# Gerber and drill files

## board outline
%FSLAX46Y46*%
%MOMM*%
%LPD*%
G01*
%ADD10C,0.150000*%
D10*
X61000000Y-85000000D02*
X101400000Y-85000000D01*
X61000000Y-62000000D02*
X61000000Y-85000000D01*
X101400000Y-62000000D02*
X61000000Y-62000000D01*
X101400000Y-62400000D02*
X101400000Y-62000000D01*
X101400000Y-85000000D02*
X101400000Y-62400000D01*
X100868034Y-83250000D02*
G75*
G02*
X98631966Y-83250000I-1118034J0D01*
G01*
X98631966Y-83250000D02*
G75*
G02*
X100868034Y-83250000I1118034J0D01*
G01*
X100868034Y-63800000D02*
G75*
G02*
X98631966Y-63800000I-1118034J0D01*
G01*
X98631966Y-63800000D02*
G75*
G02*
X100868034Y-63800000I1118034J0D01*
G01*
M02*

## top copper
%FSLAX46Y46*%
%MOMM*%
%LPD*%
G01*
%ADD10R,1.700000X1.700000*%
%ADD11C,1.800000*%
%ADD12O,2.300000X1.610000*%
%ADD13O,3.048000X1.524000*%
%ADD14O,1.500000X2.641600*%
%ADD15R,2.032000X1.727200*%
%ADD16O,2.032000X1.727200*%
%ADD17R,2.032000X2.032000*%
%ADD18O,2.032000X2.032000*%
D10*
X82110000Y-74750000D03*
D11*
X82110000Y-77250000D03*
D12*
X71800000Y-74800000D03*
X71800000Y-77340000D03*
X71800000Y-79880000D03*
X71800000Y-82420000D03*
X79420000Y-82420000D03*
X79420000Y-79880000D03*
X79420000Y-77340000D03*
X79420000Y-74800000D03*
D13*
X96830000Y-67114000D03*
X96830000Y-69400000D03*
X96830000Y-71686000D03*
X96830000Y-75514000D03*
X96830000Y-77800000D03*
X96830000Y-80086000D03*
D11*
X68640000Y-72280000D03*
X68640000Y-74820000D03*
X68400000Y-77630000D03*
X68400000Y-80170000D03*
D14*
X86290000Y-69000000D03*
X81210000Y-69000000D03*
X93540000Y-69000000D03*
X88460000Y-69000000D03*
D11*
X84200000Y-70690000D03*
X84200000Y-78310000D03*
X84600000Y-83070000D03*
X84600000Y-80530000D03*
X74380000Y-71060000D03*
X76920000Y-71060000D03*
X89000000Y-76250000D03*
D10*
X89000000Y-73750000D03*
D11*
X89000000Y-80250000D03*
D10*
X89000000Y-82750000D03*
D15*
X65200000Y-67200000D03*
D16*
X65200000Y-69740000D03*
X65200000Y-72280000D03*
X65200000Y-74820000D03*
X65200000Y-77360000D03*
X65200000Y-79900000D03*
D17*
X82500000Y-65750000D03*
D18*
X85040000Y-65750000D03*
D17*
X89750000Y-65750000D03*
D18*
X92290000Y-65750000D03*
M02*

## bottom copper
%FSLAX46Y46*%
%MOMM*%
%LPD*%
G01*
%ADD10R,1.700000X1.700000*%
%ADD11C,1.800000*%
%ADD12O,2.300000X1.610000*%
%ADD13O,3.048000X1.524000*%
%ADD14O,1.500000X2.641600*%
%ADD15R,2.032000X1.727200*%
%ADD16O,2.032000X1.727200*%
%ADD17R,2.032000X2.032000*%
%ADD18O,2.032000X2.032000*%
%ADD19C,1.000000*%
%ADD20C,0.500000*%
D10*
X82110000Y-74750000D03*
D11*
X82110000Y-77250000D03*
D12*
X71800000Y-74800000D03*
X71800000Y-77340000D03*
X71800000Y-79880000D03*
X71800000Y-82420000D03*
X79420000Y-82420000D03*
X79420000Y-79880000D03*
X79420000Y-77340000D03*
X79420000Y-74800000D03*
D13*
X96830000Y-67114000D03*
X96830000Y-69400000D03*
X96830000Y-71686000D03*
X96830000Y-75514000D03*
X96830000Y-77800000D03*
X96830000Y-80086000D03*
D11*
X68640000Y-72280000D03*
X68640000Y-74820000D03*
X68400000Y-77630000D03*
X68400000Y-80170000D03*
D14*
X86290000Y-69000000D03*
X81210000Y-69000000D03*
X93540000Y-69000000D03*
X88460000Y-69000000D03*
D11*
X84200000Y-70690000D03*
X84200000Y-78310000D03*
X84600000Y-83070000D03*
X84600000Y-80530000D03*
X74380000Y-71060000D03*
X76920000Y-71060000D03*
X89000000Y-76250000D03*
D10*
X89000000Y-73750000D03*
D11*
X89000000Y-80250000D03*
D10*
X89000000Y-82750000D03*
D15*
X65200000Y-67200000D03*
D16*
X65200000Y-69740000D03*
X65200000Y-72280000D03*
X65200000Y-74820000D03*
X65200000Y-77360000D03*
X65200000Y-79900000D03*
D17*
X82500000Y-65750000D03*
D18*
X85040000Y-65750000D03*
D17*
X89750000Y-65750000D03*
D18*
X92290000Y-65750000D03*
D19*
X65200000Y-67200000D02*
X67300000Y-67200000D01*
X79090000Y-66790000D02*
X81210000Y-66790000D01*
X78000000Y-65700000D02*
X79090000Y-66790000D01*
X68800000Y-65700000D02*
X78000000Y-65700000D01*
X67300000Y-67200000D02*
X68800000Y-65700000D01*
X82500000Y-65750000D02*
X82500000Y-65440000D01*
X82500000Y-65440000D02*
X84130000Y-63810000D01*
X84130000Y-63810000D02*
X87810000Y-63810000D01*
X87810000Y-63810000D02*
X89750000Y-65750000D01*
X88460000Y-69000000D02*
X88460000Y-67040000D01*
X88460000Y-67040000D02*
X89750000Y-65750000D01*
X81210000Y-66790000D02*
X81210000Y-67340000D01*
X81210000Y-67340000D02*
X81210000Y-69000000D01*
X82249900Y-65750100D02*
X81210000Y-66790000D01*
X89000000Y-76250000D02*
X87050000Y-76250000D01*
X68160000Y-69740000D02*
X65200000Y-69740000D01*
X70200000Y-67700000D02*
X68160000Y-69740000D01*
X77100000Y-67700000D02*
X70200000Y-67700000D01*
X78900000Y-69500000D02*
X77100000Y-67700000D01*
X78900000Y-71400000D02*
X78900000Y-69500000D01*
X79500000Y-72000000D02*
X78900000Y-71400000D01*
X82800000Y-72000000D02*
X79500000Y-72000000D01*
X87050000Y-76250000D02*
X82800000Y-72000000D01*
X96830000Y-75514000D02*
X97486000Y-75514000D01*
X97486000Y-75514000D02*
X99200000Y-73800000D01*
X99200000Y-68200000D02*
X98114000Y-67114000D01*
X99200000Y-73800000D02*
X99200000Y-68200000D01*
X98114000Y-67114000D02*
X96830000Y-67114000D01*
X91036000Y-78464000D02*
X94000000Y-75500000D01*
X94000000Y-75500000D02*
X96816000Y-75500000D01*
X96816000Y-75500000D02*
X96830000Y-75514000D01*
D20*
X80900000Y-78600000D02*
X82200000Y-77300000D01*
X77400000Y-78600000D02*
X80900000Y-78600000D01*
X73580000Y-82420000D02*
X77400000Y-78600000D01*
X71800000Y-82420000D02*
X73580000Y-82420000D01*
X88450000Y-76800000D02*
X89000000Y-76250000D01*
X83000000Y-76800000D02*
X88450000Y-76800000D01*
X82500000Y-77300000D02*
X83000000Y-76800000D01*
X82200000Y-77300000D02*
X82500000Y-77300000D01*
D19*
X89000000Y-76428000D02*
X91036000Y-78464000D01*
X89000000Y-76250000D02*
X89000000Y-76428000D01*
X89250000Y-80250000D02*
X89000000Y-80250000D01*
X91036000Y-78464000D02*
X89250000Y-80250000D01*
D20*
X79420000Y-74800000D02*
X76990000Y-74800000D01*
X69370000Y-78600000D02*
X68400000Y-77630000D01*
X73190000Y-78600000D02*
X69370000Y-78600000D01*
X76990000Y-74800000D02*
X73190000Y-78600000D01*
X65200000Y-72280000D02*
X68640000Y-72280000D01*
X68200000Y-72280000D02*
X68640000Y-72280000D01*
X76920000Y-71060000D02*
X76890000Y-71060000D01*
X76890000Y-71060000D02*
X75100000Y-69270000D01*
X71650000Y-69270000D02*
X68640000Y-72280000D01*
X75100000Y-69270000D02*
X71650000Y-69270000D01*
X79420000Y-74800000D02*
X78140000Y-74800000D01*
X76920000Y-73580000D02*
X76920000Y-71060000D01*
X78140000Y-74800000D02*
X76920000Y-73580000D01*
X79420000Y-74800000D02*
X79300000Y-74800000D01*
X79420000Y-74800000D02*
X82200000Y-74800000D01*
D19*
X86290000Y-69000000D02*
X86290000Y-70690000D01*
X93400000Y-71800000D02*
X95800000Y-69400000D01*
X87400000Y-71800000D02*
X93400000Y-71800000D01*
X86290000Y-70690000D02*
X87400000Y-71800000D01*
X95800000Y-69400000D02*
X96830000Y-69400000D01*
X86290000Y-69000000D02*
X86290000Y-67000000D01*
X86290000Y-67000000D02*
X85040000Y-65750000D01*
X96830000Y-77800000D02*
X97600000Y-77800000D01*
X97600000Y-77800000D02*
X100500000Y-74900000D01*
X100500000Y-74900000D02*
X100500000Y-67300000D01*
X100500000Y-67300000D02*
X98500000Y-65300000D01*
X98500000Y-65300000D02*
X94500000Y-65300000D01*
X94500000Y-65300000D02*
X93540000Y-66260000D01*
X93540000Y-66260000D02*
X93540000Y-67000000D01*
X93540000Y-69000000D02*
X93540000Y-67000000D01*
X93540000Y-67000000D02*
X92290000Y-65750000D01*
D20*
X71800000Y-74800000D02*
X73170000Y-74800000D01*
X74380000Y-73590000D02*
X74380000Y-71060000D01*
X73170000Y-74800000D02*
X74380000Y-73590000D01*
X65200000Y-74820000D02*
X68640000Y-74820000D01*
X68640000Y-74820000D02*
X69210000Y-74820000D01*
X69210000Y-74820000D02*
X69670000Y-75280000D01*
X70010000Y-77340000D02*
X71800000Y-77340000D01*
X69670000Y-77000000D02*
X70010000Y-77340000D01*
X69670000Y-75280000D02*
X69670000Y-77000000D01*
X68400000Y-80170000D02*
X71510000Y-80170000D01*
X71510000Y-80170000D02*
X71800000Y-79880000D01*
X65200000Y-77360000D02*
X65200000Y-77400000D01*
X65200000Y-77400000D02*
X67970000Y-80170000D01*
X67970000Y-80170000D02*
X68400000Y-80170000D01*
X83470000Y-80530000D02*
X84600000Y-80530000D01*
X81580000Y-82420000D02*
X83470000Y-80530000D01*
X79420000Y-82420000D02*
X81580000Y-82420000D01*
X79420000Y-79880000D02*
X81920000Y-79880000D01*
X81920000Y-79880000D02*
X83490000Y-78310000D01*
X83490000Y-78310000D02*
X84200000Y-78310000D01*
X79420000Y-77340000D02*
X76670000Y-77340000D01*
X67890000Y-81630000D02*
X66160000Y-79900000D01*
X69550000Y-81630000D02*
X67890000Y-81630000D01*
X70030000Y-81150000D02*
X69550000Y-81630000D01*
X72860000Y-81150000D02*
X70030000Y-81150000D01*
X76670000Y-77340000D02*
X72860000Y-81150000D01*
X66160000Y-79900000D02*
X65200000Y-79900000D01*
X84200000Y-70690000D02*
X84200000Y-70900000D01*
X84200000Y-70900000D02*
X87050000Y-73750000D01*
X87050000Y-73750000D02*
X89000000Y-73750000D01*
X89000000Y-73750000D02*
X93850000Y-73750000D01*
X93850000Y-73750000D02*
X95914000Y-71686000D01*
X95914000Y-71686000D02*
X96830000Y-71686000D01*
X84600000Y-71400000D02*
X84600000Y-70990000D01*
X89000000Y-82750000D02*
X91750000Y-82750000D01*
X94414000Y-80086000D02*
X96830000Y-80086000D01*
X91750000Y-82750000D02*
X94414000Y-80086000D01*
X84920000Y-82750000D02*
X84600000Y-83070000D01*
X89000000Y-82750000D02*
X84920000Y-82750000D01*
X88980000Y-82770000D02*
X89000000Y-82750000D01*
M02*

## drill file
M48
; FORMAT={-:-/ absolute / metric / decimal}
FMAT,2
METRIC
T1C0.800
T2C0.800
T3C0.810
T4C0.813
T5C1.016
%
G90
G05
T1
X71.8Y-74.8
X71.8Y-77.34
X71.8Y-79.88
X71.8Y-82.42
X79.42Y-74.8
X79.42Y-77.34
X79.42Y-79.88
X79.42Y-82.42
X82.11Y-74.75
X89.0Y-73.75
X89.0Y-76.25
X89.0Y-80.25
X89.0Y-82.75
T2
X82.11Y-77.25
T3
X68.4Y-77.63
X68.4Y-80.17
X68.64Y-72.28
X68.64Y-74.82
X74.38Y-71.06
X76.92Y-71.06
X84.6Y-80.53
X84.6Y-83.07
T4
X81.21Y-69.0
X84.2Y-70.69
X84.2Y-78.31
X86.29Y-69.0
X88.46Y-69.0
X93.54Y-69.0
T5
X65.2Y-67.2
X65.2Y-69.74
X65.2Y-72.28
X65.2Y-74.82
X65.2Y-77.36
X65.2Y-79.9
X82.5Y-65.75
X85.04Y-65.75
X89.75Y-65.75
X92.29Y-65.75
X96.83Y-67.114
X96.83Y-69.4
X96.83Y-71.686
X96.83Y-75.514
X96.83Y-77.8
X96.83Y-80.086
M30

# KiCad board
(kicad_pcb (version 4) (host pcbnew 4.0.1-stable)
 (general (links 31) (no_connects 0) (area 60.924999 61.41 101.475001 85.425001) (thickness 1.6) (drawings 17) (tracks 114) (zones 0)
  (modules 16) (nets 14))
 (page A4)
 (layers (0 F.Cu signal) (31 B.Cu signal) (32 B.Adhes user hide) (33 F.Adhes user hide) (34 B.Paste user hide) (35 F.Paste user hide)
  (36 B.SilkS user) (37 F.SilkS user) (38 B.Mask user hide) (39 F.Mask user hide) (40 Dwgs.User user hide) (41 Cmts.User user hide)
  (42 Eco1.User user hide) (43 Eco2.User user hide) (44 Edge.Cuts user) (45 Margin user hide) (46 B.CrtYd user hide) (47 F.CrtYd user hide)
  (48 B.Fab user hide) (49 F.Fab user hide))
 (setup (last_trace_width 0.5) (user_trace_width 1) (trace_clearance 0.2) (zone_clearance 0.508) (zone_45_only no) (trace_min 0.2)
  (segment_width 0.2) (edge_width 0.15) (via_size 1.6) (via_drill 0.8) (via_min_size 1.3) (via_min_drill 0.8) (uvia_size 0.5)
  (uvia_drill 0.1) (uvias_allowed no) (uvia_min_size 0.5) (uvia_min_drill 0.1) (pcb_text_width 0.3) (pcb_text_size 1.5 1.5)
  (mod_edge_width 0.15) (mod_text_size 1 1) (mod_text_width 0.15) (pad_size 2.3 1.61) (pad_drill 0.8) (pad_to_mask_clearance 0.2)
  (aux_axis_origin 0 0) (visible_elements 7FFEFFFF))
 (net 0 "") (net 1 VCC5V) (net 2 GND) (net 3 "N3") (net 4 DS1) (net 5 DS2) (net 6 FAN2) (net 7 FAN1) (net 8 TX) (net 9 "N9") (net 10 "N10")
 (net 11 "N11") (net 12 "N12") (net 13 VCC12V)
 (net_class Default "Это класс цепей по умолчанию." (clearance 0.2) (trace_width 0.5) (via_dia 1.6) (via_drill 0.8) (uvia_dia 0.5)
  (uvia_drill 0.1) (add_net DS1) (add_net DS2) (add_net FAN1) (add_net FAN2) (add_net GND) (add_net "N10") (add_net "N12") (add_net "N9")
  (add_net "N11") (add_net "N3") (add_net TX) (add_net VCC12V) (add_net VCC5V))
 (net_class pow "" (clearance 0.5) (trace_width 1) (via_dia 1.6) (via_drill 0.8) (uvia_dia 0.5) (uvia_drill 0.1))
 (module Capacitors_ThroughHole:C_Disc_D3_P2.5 (layer F.Cu) (at 82.11 74.75 270)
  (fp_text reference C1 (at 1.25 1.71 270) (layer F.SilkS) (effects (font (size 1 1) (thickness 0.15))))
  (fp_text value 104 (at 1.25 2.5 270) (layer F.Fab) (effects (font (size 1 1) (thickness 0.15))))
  (pad 1 thru_hole rect (at 0 0 270) (size 1.7 1.7) (drill 0.8) (layers *.Cu *.Mask F.SilkS) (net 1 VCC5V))
  (pad 2 thru_hole circle (at 2.5 0 270) (size 1.8 1.8) (drill 0.8001) (layers *.Cu *.Mask F.SilkS) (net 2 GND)))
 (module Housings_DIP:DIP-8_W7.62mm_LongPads (layer F.Cu) (at 71.8 74.8)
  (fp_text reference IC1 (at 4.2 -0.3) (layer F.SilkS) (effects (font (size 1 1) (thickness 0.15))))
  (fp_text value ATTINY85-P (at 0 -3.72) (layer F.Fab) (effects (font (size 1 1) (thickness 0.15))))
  (pad 1 thru_hole oval (at 0 0) (size 2.3 1.61) (drill 0.8) (layers *.Cu *.Mask F.SilkS) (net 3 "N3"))
  (pad 2 thru_hole oval (at 0 2.54) (size 2.3 1.61) (drill 0.8) (layers *.Cu *.Mask F.SilkS) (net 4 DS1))
  (pad 3 thru_hole oval (at 0 5.08) (size 2.3 1.61) (drill 0.8) (layers *.Cu *.Mask F.SilkS) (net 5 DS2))
  (pad 4 thru_hole oval (at 0 7.62) (size 2.3 1.61) (drill 0.8) (layers *.Cu *.Mask F.SilkS) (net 2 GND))
  (pad 5 thru_hole oval (at 7.62 7.62) (size 2.3 1.61) (drill 0.8) (layers *.Cu *.Mask F.SilkS) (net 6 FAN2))
  (pad 6 thru_hole oval (at 7.62 5.08) (size 2.3 1.61) (drill 0.8) (layers *.Cu *.Mask F.SilkS) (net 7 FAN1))
  (pad 7 thru_hole oval (at 7.62 2.54) (size 2.3 1.61) (drill 0.8) (layers *.Cu *.Mask F.SilkS) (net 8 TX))
  (pad 8 thru_hole oval (at 7.62 0) (size 2.3 1.61) (drill 0.8) (layers *.Cu *.Mask F.SilkS) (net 1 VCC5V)))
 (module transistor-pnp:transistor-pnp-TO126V (layer F.Cu) (at 98.1 69.4 270)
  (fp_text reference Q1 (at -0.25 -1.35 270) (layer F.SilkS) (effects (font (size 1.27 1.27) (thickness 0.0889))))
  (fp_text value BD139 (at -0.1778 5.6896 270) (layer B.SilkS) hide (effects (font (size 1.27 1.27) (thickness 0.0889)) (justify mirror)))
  (pad 1 thru_hole oval (at -2.286 1.27 270) (size 1.524 3.048) (drill 1.016) (layers *.Cu F.Paste F.SilkS F.Mask) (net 2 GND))
  (pad 2 thru_hole oval (at 0 1.27 270) (size 1.524 3.048) (drill 1.016) (layers *.Cu F.Paste F.SilkS F.Mask) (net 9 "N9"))
  (pad 3 thru_hole oval (at 2.286 1.27 270) (size 1.524 3.048) (drill 1.016) (layers *.Cu F.Paste F.SilkS F.Mask) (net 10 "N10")))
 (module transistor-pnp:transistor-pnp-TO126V (layer F.Cu) (at 98.1 77.8 270)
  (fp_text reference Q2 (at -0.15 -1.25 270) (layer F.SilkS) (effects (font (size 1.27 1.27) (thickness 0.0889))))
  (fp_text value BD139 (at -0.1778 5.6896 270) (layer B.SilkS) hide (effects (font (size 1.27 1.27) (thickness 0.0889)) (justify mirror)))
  (pad 1 thru_hole oval (at -2.286 1.27 270) (size 1.524 3.048) (drill 1.016) (layers *.Cu F.Paste F.SilkS F.Mask) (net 2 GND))
  (pad 2 thru_hole oval (at 0 1.27 270) (size 1.524 3.048) (drill 1.016) (layers *.Cu F.Paste F.SilkS F.Mask) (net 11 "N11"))
  (pad 3 thru_hole oval (at 2.286 1.27 270) (size 1.524 3.048) (drill 1.016) (layers *.Cu F.Paste F.SilkS F.Mask) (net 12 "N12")))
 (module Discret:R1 (layer F.Cu) (at 68.64 73.55 270)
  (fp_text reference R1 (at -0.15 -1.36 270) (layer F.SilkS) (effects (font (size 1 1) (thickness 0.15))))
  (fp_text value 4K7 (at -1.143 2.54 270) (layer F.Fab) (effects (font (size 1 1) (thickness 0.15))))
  (pad 1 thru_hole circle (at -1.27 0 270) (size 1.8 1.8) (drill 0.81) (layers *.Cu *.Mask F.SilkS) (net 1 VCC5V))
  (pad 2 thru_hole circle (at 1.27 0 270) (size 1.8 1.8) (drill 0.81) (layers *.Cu *.Mask F.SilkS) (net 4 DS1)))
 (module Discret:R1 (layer F.Cu) (at 68.4 78.9 270)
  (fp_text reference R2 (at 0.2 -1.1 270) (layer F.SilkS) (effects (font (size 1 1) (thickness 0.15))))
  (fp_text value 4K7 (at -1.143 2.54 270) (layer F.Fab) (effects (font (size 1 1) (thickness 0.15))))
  (pad 1 thru_hole circle (at -1.27 0 270) (size 1.8 1.8) (drill 0.81) (layers *.Cu *.Mask F.SilkS) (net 1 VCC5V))
  (pad 2 thru_hole circle (at 1.27 0 270) (size 1.8 1.8) (drill 0.81) (layers *.Cu *.Mask F.SilkS) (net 5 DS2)))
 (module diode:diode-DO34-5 (layer F.Cu) (at 83.75 69)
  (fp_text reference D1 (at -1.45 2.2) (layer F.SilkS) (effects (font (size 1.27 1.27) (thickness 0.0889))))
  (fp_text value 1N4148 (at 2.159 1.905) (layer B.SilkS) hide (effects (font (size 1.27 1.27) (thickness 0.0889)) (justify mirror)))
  (pad 2 thru_hole oval (at 2.54 0) (size 1.5 2.6416) (drill 0.8128) (layers *.Cu F.Paste F.SilkS F.Mask) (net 9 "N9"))
  (pad 1 thru_hole oval (at -2.54 0) (size 1.5 2.6416) (drill 0.8128) (layers *.Cu F.Paste F.SilkS F.Mask) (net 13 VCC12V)))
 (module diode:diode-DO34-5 (layer F.Cu) (at 91 69)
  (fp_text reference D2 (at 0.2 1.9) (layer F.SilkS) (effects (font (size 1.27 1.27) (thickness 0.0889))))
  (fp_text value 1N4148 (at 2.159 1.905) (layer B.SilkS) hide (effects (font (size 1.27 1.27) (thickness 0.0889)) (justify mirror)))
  (pad 2 thru_hole oval (at 2.54 0) (size 1.5 2.6416) (drill 0.8128) (layers *.Cu F.Paste F.SilkS F.Mask) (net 11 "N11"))
  (pad 1 thru_hole oval (at -2.54 0) (size 1.5 2.6416) (drill 0.8128) (layers *.Cu F.Paste F.SilkS F.Mask) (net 13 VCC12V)))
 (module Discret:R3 (layer F.Cu) (at 84.2 74.5 270)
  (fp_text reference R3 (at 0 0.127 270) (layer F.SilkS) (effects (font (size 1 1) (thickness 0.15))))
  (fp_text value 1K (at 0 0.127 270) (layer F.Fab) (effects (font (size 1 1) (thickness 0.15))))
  (pad 1 thru_hole circle (at -3.81 0 270) (size 1.8 1.8) (drill 0.8128) (layers *.Cu *.Mask F.SilkS) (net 10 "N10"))
  (pad 2 thru_hole circle (at 3.81 0 270) (size 1.8 1.8) (drill 0.8128) (layers *.Cu *.Mask F.SilkS) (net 7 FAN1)))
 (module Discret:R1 (layer F.Cu) (at 84.6 81.8 90)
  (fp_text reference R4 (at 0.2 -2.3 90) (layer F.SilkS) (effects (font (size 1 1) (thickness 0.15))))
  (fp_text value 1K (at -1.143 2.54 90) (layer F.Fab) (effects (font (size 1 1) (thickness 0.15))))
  (pad 1 thru_hole circle (at -1.27 0 90) (size 1.8 1.8) (drill 0.81) (layers *.Cu *.Mask F.SilkS) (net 12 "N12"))
  (pad 2 thru_hole circle (at 1.27 0 90) (size 1.8 1.8) (drill 0.81) (layers *.Cu *.Mask F.SilkS) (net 6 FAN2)))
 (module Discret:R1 (layer F.Cu) (at 75.65 71.06)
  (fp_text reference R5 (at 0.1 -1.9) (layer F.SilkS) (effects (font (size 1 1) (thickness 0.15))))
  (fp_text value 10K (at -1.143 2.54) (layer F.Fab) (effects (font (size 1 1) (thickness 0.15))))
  (pad 1 thru_hole circle (at -1.27 0) (size 1.8 1.8) (drill 0.81) (layers *.Cu *.Mask F.SilkS) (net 3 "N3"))
  (pad 2 thru_hole circle (at 1.27 0) (size 1.8 1.8) (drill 0.81) (layers *.Cu *.Mask F.SilkS) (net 1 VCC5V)))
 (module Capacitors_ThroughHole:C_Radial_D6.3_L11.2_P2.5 (layer F.Cu) (at 89 73.75 270)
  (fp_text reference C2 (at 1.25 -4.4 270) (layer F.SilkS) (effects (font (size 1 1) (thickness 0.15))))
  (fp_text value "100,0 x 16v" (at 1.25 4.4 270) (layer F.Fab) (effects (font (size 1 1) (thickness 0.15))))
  (pad 2 thru_hole circle (at 2.5 0 270) (size 1.8 1.8) (drill 0.8) (layers *.Cu *.Mask F.SilkS) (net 2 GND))
  (pad 1 thru_hole rect (at 0 0 270) (size 1.7 1.7) (drill 0.8) (layers *.Cu *.Mask F.SilkS) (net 10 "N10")))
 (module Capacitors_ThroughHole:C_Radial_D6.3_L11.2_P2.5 (layer F.Cu) (at 89 82.75 90)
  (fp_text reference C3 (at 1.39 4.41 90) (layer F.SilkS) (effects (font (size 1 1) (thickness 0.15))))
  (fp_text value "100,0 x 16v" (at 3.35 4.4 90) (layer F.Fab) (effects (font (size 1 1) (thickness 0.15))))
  (pad 2 thru_hole circle (at 2.5 0 90) (size 1.8 1.8) (drill 0.8) (layers *.Cu *.Mask F.SilkS) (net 2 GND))
  (pad 1 thru_hole rect (at 0 0 90) (size 1.7 1.7) (drill 0.8) (layers *.Cu *.Mask F.SilkS) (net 12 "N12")))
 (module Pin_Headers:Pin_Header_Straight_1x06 (layer F.Cu) (at 65.2 67.2)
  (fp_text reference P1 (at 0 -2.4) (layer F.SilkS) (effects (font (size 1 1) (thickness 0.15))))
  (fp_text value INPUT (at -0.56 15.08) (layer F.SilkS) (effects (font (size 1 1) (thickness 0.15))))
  (pad 1 thru_hole rect (at 0 0) (size 2.032 1.7272) (drill 1.016) (layers *.Cu *.Mask F.SilkS) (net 13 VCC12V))
  (pad 2 thru_hole oval (at 0 2.54) (size 2.032 1.7272) (drill 1.016) (layers *.Cu *.Mask F.SilkS) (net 2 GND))
  (pad 3 thru_hole oval (at 0 5.08) (size 2.032 1.7272) (drill 1.016) (layers *.Cu *.Mask F.SilkS) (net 1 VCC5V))
  (pad 4 thru_hole oval (at 0 7.62) (size 2.032 1.7272) (drill 1.016) (layers *.Cu *.Mask F.SilkS) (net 4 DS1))
  (pad 5 thru_hole oval (at 0 10.16) (size 2.032 1.7272) (drill 1.016) (layers *.Cu *.Mask F.SilkS) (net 5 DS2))
  (pad 6 thru_hole oval (at 0 12.7) (size 2.032 1.7272) (drill 1.016) (layers *.Cu *.Mask F.SilkS) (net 8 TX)))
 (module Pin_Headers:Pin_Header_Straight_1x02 (layer F.Cu) (at 82.5 65.75 90)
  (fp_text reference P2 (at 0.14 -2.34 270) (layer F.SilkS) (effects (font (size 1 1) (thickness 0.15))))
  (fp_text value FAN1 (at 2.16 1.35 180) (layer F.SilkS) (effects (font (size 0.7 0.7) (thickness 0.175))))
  (pad 1 thru_hole rect (at 0 0 90) (size 2.032 2.032) (drill 1.016) (layers *.Cu *.Mask F.SilkS) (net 13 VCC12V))
  (pad 2 thru_hole oval (at 0 2.54 90) (size 2.032 2.032) (drill 1.016) (layers *.Cu *.Mask F.SilkS) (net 9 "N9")))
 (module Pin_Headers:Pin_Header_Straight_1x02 (layer F.Cu) (at 89.75 65.75 90)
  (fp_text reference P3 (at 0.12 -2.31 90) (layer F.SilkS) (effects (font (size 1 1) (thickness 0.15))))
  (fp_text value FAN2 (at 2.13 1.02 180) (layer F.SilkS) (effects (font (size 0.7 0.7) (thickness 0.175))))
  (pad 1 thru_hole rect (at 0 0 90) (size 2.032 2.032) (drill 1.016) (layers *.Cu *.Mask F.SilkS) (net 13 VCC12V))
  (pad 2 thru_hole oval (at 0 2.54 90) (size 2.032 2.032) (drill 1.016) (layers *.Cu *.Mask F.SilkS) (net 11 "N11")))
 (gr_line (start 61 85) (end 101.4 85) (angle 90) (layer Edge.Cuts) (width 0.15))
 (gr_line (start 61 62) (end 61 85) (angle 90) (layer Edge.Cuts) (width 0.15))
 (gr_line (start 101.4 62) (end 61 62) (angle 90) (layer Edge.Cuts) (width 0.15))
 (gr_line (start 101.4 62.4) (end 101.4 62) (angle 90) (layer Edge.Cuts) (width 0.15))
 (gr_line (start 101.4 85) (end 101.4 62.4) (angle 90) (layer Edge.Cuts) (width 0.15))
 (gr_circle (center 99.75 83.25) (end 100.75 82.75) (layer Edge.Cuts) (width 0.15))
 (gr_circle (center 99.75 63.8) (end 100.75 63.3) (layer Edge.Cuts) (width 0.15))
 (segment (start 65.2 67.2) (end 67.3 67.2) (width 1) (layer B.Cu) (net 13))
 (segment (start 79.09 66.79) (end 81.21 66.79) (width 1) (layer B.Cu) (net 13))
 (segment (start 78 65.7) (end 79.09 66.79) (width 1) (layer B.Cu) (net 13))
 (segment (start 68.8 65.7) (end 78 65.7) (width 1) (layer B.Cu) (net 13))
 (segment (start 67.3 67.2) (end 68.8 65.7) (width 1) (layer B.Cu) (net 13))
 (segment (start 82.5 65.75) (end 82.5 65.44) (width 1) (layer B.Cu) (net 13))
 (segment (start 82.5 65.44) (end 84.13 63.81) (width 1) (layer B.Cu) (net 13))
 (segment (start 84.13 63.81) (end 87.81 63.81) (width 1) (layer B.Cu) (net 13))
 (segment (start 87.81 63.81) (end 89.75 65.75) (width 1) (layer B.Cu) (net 13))
 (segment (start 88.46 69) (end 88.46 67.04) (width 1) (layer B.Cu) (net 13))
 (segment (start 88.46 67.04) (end 89.75 65.75) (width 1) (layer B.Cu) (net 13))
 (segment (start 81.21 66.79) (end 81.21 67.34) (width 1) (layer B.Cu) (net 13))
 (segment (start 81.21 67.34) (end 81.21 69) (width 1) (layer B.Cu) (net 13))
 (segment (start 82.2499 65.7501) (end 81.21 66.79) (width 1) (layer B.Cu) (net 13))
 (segment (start 89 76.25) (end 87.05 76.25) (width 1) (layer B.Cu) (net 2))
 (segment (start 68.16 69.74) (end 65.2 69.74) (width 1) (layer B.Cu) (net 2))
 (segment (start 70.2 67.7) (end 68.16 69.74) (width 1) (layer B.Cu) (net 2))
 (segment (start 77.1 67.7) (end 70.2 67.7) (width 1) (layer B.Cu) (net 2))
 (segment (start 78.9 69.5) (end 77.1 67.7) (width 1) (layer B.Cu) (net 2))
 (segment (start 78.9 71.4) (end 78.9 69.5) (width 1) (layer B.Cu) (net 2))
 (segment (start 79.5 72) (end 78.9 71.4) (width 1) (layer B.Cu) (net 2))
 (segment (start 82.8 72) (end 79.5 72) (width 1) (layer B.Cu) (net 2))
 (segment (start 87.05 76.25) (end 82.8 72) (width 1) (layer B.Cu) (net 2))
 (segment (start 96.83 75.514) (end 97.486 75.514) (width 1) (layer B.Cu) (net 2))
 (segment (start 97.486 75.514) (end 99.2 73.8) (width 1) (layer B.Cu) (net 2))
 (segment (start 99.2 68.2) (end 98.114 67.114) (width 1) (layer B.Cu) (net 2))
 (segment (start 99.2 73.8) (end 99.2 68.2) (width 1) (layer B.Cu) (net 2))
 (segment (start 98.114 67.114) (end 96.83 67.114) (width 1) (layer B.Cu) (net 2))
 (segment (start 91.036 78.464) (end 94 75.5) (width 1) (layer B.Cu) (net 2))
 (segment (start 94 75.5) (end 96.816 75.5) (width 1) (layer B.Cu) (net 2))
 (segment (start 96.816 75.5) (end 96.83 75.514) (width 1) (layer B.Cu) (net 2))
 (segment (start 80.9 78.6) (end 82.2 77.3) (width 0.5) (layer B.Cu) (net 2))
 (segment (start 77.4 78.6) (end 80.9 78.6) (width 0.5) (layer B.Cu) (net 2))
 (segment (start 73.58 82.42) (end 77.4 78.6) (width 0.5) (layer B.Cu) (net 2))
 (segment (start 71.8 82.42) (end 73.58 82.42) (width 0.5) (layer B.Cu) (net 2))
 (segment (start 88.45 76.8) (end 89 76.25) (width 0.5) (layer B.Cu) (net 2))
 (segment (start 83 76.8) (end 88.45 76.8) (width 0.5) (layer B.Cu) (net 2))
 (segment (start 82.5 77.3) (end 83 76.8) (width 0.5) (layer B.Cu) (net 2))
 (segment (start 82.2 77.3) (end 82.5 77.3) (width 0.5) (layer B.Cu) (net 2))
 (segment (start 89 76.428) (end 91.036 78.464) (width 1) (layer B.Cu) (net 2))
 (segment (start 89 76.25) (end 89 76.428) (width 1) (layer B.Cu) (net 2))
 (segment (start 89.25 80.25) (end 89 80.25) (width 1) (layer B.Cu) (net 2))
 (segment (start 91.036 78.464) (end 89.25 80.25) (width 1) (layer B.Cu) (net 2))
 (segment (start 79.42 74.8) (end 76.99 74.8) (width 0.5) (layer B.Cu) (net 1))
 (segment (start 69.37 78.6) (end 68.4 77.63) (width 0.5) (layer B.Cu) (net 1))
 (segment (start 73.19 78.6) (end 69.37 78.6) (width 0.5) (layer B.Cu) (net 1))
 (segment (start 76.99 74.8) (end 73.19 78.6) (width 0.5) (layer B.Cu) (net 1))
 (segment (start 65.2 72.28) (end 68.64 72.28) (width 0.5) (layer B.Cu) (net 1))
 (segment (start 68.2 72.28) (end 68.64 72.28) (width 0.5) (layer B.Cu) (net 1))
 (segment (start 76.92 71.06) (end 76.89 71.06) (width 0.5) (layer B.Cu) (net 1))
 (segment (start 76.89 71.06) (end 75.1 69.27) (width 0.5) (layer B.Cu) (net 1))
 (segment (start 71.65 69.27) (end 68.64 72.28) (width 0.5) (layer B.Cu) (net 1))
 (segment (start 75.1 69.27) (end 71.65 69.27) (width 0.5) (layer B.Cu) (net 1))
 (segment (start 79.42 74.8) (end 78.14 74.8) (width 0.5) (layer B.Cu) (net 1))
 (segment (start 76.92 73.58) (end 76.92 71.06) (width 0.5) (layer B.Cu) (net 1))
 (segment (start 78.14 74.8) (end 76.92 73.58) (width 0.5) (layer B.Cu) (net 1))
 (segment (start 79.42 74.8) (end 79.3 74.8) (width 0.5) (layer B.Cu) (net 1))
 (segment (start 79.42 74.8) (end 82.2 74.8) (width 0.5) (layer B.Cu) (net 1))
 (segment (start 86.29 69) (end 86.29 70.69) (width 1) (layer B.Cu) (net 9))
 (segment (start 93.4 71.8) (end 95.8 69.4) (width 1) (layer B.Cu) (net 9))
 (segment (start 87.4 71.8) (end 93.4 71.8) (width 1) (layer B.Cu) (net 9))
 (segment (start 86.29 70.69) (end 87.4 71.8) (width 1) (layer B.Cu) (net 9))
 (segment (start 95.8 69.4) (end 96.83 69.4) (width 1) (layer B.Cu) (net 9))
 (segment (start 86.29 69) (end 86.29 67) (width 1) (layer B.Cu) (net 9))
 (segment (start 86.29 67) (end 85.04 65.75) (width 1) (layer B.Cu) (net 9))
 (segment (start 96.83 77.8) (end 97.6 77.8) (width 1) (layer B.Cu) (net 11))
 (segment (start 97.6 77.8) (end 100.5 74.9) (width 1) (layer B.Cu) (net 11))
 (segment (start 100.5 74.9) (end 100.5 67.3) (width 1) (layer B.Cu) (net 11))
 (segment (start 100.5 67.3) (end 98.5 65.3) (width 1) (layer B.Cu) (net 11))
 (segment (start 98.5 65.3) (end 94.5 65.3) (width 1) (layer B.Cu) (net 11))
 (segment (start 94.5 65.3) (end 93.54 66.26) (width 1) (layer B.Cu) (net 11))
 (segment (start 93.54 66.26) (end 93.54 67) (width 1) (layer B.Cu) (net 11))
 (segment (start 93.54 69) (end 93.54 67) (width 1) (layer B.Cu) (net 11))
 (segment (start 93.54 67) (end 92.29 65.75) (width 1) (layer B.Cu) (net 11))
 (segment (start 71.8 74.8) (end 73.17 74.8) (width 0.5) (layer B.Cu) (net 3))
 (segment (start 74.38 73.59) (end 74.38 71.06) (width 0.5) (layer B.Cu) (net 3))
 (segment (start 73.17 74.8) (end 74.38 73.59) (width 0.5) (layer B.Cu) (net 3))
 (segment (start 65.2 74.82) (end 68.64 74.82) (width 0.5) (layer B.Cu) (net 4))
 (segment (start 68.64 74.82) (end 69.21 74.82) (width 0.5) (layer B.Cu) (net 4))
 (segment (start 69.21 74.82) (end 69.67 75.28) (width 0.5) (layer B.Cu) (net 4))
 (segment (start 70.01 77.34) (end 71.8 77.34) (width 0.5) (layer B.Cu) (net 4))
 (segment (start 69.67 77) (end 70.01 77.34) (width 0.5) (layer B.Cu) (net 4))
 (segment (start 69.67 75.28) (end 69.67 77) (width 0.5) (layer B.Cu) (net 4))
 (segment (start 68.4 80.17) (end 71.51 80.17) (width 0.5) (layer B.Cu) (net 5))
 (segment (start 71.51 80.17) (end 71.8 79.88) (width 0.5) (layer B.Cu) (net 5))
 (segment (start 65.2 77.36) (end 65.2 77.4) (width 0.5) (layer B.Cu) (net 5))
 (segment (start 65.2 77.4) (end 67.97 80.17) (width 0.5) (layer B.Cu) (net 5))
 (segment (start 67.97 80.17) (end 68.4 80.17) (width 0.5) (layer B.Cu) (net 5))
 (segment (start 83.47 80.53) (end 84.6 80.53) (width 0.5) (layer B.Cu) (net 6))
 (segment (start 81.58 82.42) (end 83.47 80.53) (width 0.5) (layer B.Cu) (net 6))
 (segment (start 79.42 82.42) (end 81.58 82.42) (width 0.5) (layer B.Cu) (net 6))
 (segment (start 79.42 79.88) (end 81.92 79.88) (width 0.5) (layer B.Cu) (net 7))
 (segment (start 81.92 79.88) (end 83.49 78.31) (width 0.5) (layer B.Cu) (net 7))
 (segment (start 83.49 78.31) (end 84.2 78.31) (width 0.5) (layer B.Cu) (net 7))
 (segment (start 79.42 77.34) (end 76.67 77.34) (width 0.5) (layer B.Cu) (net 8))
 (segment (start 67.89 81.63) (end 66.16 79.9) (width 0.5) (layer B.Cu) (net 8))
 (segment (start 69.55 81.63) (end 67.89 81.63) (width 0.5) (layer B.Cu) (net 8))
 (segment (start 70.03 81.15) (end 69.55 81.63) (width 0.5) (layer B.Cu) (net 8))
 (segment (start 72.86 81.15) (end 70.03 81.15) (width 0.5) (layer B.Cu) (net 8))
 (segment (start 76.67 77.34) (end 72.86 81.15) (width 0.5) (layer B.Cu) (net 8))
 (segment (start 66.16 79.9) (end 65.2 79.9) (width 0.5) (layer B.Cu) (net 8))
 (segment (start 84.2 70.69) (end 84.2 70.9) (width 0.5) (layer B.Cu) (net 10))
 (segment (start 84.2 70.9) (end 87.05 73.75) (width 0.5) (layer B.Cu) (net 10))
 (segment (start 87.05 73.75) (end 89 73.75) (width 0.5) (layer B.Cu) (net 10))
 (segment (start 89 73.75) (end 93.85 73.75) (width 0.5) (layer B.Cu) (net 10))
 (segment (start 93.85 73.75) (end 95.914 71.686) (width 0.5) (layer B.Cu) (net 10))
 (segment (start 95.914 71.686) (end 96.83 71.686) (width 0.5) (layer B.Cu) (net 10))
 (segment (start 84.6 71.4) (end 84.6 70.99) (width 0.5) (layer B.Cu) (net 10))
 (segment (start 89 82.75) (end 91.75 82.75) (width 0.5) (layer B.Cu) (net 12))
 (segment (start 94.414 80.086) (end 96.83 80.086) (width 0.5) (layer B.Cu) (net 12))
 (segment (start 91.75 82.75) (end 94.414 80.086) (width 0.5) (layer B.Cu) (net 12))
 (segment (start 84.92 82.75) (end 84.6 83.07) (width 0.5) (layer B.Cu) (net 12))
 (segment (start 89 82.75) (end 84.92 82.75) (width 0.5) (layer B.Cu) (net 12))
 (segment (start 88.98 82.77) (end 89 82.75) (width 0.5) (layer B.Cu) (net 12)))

